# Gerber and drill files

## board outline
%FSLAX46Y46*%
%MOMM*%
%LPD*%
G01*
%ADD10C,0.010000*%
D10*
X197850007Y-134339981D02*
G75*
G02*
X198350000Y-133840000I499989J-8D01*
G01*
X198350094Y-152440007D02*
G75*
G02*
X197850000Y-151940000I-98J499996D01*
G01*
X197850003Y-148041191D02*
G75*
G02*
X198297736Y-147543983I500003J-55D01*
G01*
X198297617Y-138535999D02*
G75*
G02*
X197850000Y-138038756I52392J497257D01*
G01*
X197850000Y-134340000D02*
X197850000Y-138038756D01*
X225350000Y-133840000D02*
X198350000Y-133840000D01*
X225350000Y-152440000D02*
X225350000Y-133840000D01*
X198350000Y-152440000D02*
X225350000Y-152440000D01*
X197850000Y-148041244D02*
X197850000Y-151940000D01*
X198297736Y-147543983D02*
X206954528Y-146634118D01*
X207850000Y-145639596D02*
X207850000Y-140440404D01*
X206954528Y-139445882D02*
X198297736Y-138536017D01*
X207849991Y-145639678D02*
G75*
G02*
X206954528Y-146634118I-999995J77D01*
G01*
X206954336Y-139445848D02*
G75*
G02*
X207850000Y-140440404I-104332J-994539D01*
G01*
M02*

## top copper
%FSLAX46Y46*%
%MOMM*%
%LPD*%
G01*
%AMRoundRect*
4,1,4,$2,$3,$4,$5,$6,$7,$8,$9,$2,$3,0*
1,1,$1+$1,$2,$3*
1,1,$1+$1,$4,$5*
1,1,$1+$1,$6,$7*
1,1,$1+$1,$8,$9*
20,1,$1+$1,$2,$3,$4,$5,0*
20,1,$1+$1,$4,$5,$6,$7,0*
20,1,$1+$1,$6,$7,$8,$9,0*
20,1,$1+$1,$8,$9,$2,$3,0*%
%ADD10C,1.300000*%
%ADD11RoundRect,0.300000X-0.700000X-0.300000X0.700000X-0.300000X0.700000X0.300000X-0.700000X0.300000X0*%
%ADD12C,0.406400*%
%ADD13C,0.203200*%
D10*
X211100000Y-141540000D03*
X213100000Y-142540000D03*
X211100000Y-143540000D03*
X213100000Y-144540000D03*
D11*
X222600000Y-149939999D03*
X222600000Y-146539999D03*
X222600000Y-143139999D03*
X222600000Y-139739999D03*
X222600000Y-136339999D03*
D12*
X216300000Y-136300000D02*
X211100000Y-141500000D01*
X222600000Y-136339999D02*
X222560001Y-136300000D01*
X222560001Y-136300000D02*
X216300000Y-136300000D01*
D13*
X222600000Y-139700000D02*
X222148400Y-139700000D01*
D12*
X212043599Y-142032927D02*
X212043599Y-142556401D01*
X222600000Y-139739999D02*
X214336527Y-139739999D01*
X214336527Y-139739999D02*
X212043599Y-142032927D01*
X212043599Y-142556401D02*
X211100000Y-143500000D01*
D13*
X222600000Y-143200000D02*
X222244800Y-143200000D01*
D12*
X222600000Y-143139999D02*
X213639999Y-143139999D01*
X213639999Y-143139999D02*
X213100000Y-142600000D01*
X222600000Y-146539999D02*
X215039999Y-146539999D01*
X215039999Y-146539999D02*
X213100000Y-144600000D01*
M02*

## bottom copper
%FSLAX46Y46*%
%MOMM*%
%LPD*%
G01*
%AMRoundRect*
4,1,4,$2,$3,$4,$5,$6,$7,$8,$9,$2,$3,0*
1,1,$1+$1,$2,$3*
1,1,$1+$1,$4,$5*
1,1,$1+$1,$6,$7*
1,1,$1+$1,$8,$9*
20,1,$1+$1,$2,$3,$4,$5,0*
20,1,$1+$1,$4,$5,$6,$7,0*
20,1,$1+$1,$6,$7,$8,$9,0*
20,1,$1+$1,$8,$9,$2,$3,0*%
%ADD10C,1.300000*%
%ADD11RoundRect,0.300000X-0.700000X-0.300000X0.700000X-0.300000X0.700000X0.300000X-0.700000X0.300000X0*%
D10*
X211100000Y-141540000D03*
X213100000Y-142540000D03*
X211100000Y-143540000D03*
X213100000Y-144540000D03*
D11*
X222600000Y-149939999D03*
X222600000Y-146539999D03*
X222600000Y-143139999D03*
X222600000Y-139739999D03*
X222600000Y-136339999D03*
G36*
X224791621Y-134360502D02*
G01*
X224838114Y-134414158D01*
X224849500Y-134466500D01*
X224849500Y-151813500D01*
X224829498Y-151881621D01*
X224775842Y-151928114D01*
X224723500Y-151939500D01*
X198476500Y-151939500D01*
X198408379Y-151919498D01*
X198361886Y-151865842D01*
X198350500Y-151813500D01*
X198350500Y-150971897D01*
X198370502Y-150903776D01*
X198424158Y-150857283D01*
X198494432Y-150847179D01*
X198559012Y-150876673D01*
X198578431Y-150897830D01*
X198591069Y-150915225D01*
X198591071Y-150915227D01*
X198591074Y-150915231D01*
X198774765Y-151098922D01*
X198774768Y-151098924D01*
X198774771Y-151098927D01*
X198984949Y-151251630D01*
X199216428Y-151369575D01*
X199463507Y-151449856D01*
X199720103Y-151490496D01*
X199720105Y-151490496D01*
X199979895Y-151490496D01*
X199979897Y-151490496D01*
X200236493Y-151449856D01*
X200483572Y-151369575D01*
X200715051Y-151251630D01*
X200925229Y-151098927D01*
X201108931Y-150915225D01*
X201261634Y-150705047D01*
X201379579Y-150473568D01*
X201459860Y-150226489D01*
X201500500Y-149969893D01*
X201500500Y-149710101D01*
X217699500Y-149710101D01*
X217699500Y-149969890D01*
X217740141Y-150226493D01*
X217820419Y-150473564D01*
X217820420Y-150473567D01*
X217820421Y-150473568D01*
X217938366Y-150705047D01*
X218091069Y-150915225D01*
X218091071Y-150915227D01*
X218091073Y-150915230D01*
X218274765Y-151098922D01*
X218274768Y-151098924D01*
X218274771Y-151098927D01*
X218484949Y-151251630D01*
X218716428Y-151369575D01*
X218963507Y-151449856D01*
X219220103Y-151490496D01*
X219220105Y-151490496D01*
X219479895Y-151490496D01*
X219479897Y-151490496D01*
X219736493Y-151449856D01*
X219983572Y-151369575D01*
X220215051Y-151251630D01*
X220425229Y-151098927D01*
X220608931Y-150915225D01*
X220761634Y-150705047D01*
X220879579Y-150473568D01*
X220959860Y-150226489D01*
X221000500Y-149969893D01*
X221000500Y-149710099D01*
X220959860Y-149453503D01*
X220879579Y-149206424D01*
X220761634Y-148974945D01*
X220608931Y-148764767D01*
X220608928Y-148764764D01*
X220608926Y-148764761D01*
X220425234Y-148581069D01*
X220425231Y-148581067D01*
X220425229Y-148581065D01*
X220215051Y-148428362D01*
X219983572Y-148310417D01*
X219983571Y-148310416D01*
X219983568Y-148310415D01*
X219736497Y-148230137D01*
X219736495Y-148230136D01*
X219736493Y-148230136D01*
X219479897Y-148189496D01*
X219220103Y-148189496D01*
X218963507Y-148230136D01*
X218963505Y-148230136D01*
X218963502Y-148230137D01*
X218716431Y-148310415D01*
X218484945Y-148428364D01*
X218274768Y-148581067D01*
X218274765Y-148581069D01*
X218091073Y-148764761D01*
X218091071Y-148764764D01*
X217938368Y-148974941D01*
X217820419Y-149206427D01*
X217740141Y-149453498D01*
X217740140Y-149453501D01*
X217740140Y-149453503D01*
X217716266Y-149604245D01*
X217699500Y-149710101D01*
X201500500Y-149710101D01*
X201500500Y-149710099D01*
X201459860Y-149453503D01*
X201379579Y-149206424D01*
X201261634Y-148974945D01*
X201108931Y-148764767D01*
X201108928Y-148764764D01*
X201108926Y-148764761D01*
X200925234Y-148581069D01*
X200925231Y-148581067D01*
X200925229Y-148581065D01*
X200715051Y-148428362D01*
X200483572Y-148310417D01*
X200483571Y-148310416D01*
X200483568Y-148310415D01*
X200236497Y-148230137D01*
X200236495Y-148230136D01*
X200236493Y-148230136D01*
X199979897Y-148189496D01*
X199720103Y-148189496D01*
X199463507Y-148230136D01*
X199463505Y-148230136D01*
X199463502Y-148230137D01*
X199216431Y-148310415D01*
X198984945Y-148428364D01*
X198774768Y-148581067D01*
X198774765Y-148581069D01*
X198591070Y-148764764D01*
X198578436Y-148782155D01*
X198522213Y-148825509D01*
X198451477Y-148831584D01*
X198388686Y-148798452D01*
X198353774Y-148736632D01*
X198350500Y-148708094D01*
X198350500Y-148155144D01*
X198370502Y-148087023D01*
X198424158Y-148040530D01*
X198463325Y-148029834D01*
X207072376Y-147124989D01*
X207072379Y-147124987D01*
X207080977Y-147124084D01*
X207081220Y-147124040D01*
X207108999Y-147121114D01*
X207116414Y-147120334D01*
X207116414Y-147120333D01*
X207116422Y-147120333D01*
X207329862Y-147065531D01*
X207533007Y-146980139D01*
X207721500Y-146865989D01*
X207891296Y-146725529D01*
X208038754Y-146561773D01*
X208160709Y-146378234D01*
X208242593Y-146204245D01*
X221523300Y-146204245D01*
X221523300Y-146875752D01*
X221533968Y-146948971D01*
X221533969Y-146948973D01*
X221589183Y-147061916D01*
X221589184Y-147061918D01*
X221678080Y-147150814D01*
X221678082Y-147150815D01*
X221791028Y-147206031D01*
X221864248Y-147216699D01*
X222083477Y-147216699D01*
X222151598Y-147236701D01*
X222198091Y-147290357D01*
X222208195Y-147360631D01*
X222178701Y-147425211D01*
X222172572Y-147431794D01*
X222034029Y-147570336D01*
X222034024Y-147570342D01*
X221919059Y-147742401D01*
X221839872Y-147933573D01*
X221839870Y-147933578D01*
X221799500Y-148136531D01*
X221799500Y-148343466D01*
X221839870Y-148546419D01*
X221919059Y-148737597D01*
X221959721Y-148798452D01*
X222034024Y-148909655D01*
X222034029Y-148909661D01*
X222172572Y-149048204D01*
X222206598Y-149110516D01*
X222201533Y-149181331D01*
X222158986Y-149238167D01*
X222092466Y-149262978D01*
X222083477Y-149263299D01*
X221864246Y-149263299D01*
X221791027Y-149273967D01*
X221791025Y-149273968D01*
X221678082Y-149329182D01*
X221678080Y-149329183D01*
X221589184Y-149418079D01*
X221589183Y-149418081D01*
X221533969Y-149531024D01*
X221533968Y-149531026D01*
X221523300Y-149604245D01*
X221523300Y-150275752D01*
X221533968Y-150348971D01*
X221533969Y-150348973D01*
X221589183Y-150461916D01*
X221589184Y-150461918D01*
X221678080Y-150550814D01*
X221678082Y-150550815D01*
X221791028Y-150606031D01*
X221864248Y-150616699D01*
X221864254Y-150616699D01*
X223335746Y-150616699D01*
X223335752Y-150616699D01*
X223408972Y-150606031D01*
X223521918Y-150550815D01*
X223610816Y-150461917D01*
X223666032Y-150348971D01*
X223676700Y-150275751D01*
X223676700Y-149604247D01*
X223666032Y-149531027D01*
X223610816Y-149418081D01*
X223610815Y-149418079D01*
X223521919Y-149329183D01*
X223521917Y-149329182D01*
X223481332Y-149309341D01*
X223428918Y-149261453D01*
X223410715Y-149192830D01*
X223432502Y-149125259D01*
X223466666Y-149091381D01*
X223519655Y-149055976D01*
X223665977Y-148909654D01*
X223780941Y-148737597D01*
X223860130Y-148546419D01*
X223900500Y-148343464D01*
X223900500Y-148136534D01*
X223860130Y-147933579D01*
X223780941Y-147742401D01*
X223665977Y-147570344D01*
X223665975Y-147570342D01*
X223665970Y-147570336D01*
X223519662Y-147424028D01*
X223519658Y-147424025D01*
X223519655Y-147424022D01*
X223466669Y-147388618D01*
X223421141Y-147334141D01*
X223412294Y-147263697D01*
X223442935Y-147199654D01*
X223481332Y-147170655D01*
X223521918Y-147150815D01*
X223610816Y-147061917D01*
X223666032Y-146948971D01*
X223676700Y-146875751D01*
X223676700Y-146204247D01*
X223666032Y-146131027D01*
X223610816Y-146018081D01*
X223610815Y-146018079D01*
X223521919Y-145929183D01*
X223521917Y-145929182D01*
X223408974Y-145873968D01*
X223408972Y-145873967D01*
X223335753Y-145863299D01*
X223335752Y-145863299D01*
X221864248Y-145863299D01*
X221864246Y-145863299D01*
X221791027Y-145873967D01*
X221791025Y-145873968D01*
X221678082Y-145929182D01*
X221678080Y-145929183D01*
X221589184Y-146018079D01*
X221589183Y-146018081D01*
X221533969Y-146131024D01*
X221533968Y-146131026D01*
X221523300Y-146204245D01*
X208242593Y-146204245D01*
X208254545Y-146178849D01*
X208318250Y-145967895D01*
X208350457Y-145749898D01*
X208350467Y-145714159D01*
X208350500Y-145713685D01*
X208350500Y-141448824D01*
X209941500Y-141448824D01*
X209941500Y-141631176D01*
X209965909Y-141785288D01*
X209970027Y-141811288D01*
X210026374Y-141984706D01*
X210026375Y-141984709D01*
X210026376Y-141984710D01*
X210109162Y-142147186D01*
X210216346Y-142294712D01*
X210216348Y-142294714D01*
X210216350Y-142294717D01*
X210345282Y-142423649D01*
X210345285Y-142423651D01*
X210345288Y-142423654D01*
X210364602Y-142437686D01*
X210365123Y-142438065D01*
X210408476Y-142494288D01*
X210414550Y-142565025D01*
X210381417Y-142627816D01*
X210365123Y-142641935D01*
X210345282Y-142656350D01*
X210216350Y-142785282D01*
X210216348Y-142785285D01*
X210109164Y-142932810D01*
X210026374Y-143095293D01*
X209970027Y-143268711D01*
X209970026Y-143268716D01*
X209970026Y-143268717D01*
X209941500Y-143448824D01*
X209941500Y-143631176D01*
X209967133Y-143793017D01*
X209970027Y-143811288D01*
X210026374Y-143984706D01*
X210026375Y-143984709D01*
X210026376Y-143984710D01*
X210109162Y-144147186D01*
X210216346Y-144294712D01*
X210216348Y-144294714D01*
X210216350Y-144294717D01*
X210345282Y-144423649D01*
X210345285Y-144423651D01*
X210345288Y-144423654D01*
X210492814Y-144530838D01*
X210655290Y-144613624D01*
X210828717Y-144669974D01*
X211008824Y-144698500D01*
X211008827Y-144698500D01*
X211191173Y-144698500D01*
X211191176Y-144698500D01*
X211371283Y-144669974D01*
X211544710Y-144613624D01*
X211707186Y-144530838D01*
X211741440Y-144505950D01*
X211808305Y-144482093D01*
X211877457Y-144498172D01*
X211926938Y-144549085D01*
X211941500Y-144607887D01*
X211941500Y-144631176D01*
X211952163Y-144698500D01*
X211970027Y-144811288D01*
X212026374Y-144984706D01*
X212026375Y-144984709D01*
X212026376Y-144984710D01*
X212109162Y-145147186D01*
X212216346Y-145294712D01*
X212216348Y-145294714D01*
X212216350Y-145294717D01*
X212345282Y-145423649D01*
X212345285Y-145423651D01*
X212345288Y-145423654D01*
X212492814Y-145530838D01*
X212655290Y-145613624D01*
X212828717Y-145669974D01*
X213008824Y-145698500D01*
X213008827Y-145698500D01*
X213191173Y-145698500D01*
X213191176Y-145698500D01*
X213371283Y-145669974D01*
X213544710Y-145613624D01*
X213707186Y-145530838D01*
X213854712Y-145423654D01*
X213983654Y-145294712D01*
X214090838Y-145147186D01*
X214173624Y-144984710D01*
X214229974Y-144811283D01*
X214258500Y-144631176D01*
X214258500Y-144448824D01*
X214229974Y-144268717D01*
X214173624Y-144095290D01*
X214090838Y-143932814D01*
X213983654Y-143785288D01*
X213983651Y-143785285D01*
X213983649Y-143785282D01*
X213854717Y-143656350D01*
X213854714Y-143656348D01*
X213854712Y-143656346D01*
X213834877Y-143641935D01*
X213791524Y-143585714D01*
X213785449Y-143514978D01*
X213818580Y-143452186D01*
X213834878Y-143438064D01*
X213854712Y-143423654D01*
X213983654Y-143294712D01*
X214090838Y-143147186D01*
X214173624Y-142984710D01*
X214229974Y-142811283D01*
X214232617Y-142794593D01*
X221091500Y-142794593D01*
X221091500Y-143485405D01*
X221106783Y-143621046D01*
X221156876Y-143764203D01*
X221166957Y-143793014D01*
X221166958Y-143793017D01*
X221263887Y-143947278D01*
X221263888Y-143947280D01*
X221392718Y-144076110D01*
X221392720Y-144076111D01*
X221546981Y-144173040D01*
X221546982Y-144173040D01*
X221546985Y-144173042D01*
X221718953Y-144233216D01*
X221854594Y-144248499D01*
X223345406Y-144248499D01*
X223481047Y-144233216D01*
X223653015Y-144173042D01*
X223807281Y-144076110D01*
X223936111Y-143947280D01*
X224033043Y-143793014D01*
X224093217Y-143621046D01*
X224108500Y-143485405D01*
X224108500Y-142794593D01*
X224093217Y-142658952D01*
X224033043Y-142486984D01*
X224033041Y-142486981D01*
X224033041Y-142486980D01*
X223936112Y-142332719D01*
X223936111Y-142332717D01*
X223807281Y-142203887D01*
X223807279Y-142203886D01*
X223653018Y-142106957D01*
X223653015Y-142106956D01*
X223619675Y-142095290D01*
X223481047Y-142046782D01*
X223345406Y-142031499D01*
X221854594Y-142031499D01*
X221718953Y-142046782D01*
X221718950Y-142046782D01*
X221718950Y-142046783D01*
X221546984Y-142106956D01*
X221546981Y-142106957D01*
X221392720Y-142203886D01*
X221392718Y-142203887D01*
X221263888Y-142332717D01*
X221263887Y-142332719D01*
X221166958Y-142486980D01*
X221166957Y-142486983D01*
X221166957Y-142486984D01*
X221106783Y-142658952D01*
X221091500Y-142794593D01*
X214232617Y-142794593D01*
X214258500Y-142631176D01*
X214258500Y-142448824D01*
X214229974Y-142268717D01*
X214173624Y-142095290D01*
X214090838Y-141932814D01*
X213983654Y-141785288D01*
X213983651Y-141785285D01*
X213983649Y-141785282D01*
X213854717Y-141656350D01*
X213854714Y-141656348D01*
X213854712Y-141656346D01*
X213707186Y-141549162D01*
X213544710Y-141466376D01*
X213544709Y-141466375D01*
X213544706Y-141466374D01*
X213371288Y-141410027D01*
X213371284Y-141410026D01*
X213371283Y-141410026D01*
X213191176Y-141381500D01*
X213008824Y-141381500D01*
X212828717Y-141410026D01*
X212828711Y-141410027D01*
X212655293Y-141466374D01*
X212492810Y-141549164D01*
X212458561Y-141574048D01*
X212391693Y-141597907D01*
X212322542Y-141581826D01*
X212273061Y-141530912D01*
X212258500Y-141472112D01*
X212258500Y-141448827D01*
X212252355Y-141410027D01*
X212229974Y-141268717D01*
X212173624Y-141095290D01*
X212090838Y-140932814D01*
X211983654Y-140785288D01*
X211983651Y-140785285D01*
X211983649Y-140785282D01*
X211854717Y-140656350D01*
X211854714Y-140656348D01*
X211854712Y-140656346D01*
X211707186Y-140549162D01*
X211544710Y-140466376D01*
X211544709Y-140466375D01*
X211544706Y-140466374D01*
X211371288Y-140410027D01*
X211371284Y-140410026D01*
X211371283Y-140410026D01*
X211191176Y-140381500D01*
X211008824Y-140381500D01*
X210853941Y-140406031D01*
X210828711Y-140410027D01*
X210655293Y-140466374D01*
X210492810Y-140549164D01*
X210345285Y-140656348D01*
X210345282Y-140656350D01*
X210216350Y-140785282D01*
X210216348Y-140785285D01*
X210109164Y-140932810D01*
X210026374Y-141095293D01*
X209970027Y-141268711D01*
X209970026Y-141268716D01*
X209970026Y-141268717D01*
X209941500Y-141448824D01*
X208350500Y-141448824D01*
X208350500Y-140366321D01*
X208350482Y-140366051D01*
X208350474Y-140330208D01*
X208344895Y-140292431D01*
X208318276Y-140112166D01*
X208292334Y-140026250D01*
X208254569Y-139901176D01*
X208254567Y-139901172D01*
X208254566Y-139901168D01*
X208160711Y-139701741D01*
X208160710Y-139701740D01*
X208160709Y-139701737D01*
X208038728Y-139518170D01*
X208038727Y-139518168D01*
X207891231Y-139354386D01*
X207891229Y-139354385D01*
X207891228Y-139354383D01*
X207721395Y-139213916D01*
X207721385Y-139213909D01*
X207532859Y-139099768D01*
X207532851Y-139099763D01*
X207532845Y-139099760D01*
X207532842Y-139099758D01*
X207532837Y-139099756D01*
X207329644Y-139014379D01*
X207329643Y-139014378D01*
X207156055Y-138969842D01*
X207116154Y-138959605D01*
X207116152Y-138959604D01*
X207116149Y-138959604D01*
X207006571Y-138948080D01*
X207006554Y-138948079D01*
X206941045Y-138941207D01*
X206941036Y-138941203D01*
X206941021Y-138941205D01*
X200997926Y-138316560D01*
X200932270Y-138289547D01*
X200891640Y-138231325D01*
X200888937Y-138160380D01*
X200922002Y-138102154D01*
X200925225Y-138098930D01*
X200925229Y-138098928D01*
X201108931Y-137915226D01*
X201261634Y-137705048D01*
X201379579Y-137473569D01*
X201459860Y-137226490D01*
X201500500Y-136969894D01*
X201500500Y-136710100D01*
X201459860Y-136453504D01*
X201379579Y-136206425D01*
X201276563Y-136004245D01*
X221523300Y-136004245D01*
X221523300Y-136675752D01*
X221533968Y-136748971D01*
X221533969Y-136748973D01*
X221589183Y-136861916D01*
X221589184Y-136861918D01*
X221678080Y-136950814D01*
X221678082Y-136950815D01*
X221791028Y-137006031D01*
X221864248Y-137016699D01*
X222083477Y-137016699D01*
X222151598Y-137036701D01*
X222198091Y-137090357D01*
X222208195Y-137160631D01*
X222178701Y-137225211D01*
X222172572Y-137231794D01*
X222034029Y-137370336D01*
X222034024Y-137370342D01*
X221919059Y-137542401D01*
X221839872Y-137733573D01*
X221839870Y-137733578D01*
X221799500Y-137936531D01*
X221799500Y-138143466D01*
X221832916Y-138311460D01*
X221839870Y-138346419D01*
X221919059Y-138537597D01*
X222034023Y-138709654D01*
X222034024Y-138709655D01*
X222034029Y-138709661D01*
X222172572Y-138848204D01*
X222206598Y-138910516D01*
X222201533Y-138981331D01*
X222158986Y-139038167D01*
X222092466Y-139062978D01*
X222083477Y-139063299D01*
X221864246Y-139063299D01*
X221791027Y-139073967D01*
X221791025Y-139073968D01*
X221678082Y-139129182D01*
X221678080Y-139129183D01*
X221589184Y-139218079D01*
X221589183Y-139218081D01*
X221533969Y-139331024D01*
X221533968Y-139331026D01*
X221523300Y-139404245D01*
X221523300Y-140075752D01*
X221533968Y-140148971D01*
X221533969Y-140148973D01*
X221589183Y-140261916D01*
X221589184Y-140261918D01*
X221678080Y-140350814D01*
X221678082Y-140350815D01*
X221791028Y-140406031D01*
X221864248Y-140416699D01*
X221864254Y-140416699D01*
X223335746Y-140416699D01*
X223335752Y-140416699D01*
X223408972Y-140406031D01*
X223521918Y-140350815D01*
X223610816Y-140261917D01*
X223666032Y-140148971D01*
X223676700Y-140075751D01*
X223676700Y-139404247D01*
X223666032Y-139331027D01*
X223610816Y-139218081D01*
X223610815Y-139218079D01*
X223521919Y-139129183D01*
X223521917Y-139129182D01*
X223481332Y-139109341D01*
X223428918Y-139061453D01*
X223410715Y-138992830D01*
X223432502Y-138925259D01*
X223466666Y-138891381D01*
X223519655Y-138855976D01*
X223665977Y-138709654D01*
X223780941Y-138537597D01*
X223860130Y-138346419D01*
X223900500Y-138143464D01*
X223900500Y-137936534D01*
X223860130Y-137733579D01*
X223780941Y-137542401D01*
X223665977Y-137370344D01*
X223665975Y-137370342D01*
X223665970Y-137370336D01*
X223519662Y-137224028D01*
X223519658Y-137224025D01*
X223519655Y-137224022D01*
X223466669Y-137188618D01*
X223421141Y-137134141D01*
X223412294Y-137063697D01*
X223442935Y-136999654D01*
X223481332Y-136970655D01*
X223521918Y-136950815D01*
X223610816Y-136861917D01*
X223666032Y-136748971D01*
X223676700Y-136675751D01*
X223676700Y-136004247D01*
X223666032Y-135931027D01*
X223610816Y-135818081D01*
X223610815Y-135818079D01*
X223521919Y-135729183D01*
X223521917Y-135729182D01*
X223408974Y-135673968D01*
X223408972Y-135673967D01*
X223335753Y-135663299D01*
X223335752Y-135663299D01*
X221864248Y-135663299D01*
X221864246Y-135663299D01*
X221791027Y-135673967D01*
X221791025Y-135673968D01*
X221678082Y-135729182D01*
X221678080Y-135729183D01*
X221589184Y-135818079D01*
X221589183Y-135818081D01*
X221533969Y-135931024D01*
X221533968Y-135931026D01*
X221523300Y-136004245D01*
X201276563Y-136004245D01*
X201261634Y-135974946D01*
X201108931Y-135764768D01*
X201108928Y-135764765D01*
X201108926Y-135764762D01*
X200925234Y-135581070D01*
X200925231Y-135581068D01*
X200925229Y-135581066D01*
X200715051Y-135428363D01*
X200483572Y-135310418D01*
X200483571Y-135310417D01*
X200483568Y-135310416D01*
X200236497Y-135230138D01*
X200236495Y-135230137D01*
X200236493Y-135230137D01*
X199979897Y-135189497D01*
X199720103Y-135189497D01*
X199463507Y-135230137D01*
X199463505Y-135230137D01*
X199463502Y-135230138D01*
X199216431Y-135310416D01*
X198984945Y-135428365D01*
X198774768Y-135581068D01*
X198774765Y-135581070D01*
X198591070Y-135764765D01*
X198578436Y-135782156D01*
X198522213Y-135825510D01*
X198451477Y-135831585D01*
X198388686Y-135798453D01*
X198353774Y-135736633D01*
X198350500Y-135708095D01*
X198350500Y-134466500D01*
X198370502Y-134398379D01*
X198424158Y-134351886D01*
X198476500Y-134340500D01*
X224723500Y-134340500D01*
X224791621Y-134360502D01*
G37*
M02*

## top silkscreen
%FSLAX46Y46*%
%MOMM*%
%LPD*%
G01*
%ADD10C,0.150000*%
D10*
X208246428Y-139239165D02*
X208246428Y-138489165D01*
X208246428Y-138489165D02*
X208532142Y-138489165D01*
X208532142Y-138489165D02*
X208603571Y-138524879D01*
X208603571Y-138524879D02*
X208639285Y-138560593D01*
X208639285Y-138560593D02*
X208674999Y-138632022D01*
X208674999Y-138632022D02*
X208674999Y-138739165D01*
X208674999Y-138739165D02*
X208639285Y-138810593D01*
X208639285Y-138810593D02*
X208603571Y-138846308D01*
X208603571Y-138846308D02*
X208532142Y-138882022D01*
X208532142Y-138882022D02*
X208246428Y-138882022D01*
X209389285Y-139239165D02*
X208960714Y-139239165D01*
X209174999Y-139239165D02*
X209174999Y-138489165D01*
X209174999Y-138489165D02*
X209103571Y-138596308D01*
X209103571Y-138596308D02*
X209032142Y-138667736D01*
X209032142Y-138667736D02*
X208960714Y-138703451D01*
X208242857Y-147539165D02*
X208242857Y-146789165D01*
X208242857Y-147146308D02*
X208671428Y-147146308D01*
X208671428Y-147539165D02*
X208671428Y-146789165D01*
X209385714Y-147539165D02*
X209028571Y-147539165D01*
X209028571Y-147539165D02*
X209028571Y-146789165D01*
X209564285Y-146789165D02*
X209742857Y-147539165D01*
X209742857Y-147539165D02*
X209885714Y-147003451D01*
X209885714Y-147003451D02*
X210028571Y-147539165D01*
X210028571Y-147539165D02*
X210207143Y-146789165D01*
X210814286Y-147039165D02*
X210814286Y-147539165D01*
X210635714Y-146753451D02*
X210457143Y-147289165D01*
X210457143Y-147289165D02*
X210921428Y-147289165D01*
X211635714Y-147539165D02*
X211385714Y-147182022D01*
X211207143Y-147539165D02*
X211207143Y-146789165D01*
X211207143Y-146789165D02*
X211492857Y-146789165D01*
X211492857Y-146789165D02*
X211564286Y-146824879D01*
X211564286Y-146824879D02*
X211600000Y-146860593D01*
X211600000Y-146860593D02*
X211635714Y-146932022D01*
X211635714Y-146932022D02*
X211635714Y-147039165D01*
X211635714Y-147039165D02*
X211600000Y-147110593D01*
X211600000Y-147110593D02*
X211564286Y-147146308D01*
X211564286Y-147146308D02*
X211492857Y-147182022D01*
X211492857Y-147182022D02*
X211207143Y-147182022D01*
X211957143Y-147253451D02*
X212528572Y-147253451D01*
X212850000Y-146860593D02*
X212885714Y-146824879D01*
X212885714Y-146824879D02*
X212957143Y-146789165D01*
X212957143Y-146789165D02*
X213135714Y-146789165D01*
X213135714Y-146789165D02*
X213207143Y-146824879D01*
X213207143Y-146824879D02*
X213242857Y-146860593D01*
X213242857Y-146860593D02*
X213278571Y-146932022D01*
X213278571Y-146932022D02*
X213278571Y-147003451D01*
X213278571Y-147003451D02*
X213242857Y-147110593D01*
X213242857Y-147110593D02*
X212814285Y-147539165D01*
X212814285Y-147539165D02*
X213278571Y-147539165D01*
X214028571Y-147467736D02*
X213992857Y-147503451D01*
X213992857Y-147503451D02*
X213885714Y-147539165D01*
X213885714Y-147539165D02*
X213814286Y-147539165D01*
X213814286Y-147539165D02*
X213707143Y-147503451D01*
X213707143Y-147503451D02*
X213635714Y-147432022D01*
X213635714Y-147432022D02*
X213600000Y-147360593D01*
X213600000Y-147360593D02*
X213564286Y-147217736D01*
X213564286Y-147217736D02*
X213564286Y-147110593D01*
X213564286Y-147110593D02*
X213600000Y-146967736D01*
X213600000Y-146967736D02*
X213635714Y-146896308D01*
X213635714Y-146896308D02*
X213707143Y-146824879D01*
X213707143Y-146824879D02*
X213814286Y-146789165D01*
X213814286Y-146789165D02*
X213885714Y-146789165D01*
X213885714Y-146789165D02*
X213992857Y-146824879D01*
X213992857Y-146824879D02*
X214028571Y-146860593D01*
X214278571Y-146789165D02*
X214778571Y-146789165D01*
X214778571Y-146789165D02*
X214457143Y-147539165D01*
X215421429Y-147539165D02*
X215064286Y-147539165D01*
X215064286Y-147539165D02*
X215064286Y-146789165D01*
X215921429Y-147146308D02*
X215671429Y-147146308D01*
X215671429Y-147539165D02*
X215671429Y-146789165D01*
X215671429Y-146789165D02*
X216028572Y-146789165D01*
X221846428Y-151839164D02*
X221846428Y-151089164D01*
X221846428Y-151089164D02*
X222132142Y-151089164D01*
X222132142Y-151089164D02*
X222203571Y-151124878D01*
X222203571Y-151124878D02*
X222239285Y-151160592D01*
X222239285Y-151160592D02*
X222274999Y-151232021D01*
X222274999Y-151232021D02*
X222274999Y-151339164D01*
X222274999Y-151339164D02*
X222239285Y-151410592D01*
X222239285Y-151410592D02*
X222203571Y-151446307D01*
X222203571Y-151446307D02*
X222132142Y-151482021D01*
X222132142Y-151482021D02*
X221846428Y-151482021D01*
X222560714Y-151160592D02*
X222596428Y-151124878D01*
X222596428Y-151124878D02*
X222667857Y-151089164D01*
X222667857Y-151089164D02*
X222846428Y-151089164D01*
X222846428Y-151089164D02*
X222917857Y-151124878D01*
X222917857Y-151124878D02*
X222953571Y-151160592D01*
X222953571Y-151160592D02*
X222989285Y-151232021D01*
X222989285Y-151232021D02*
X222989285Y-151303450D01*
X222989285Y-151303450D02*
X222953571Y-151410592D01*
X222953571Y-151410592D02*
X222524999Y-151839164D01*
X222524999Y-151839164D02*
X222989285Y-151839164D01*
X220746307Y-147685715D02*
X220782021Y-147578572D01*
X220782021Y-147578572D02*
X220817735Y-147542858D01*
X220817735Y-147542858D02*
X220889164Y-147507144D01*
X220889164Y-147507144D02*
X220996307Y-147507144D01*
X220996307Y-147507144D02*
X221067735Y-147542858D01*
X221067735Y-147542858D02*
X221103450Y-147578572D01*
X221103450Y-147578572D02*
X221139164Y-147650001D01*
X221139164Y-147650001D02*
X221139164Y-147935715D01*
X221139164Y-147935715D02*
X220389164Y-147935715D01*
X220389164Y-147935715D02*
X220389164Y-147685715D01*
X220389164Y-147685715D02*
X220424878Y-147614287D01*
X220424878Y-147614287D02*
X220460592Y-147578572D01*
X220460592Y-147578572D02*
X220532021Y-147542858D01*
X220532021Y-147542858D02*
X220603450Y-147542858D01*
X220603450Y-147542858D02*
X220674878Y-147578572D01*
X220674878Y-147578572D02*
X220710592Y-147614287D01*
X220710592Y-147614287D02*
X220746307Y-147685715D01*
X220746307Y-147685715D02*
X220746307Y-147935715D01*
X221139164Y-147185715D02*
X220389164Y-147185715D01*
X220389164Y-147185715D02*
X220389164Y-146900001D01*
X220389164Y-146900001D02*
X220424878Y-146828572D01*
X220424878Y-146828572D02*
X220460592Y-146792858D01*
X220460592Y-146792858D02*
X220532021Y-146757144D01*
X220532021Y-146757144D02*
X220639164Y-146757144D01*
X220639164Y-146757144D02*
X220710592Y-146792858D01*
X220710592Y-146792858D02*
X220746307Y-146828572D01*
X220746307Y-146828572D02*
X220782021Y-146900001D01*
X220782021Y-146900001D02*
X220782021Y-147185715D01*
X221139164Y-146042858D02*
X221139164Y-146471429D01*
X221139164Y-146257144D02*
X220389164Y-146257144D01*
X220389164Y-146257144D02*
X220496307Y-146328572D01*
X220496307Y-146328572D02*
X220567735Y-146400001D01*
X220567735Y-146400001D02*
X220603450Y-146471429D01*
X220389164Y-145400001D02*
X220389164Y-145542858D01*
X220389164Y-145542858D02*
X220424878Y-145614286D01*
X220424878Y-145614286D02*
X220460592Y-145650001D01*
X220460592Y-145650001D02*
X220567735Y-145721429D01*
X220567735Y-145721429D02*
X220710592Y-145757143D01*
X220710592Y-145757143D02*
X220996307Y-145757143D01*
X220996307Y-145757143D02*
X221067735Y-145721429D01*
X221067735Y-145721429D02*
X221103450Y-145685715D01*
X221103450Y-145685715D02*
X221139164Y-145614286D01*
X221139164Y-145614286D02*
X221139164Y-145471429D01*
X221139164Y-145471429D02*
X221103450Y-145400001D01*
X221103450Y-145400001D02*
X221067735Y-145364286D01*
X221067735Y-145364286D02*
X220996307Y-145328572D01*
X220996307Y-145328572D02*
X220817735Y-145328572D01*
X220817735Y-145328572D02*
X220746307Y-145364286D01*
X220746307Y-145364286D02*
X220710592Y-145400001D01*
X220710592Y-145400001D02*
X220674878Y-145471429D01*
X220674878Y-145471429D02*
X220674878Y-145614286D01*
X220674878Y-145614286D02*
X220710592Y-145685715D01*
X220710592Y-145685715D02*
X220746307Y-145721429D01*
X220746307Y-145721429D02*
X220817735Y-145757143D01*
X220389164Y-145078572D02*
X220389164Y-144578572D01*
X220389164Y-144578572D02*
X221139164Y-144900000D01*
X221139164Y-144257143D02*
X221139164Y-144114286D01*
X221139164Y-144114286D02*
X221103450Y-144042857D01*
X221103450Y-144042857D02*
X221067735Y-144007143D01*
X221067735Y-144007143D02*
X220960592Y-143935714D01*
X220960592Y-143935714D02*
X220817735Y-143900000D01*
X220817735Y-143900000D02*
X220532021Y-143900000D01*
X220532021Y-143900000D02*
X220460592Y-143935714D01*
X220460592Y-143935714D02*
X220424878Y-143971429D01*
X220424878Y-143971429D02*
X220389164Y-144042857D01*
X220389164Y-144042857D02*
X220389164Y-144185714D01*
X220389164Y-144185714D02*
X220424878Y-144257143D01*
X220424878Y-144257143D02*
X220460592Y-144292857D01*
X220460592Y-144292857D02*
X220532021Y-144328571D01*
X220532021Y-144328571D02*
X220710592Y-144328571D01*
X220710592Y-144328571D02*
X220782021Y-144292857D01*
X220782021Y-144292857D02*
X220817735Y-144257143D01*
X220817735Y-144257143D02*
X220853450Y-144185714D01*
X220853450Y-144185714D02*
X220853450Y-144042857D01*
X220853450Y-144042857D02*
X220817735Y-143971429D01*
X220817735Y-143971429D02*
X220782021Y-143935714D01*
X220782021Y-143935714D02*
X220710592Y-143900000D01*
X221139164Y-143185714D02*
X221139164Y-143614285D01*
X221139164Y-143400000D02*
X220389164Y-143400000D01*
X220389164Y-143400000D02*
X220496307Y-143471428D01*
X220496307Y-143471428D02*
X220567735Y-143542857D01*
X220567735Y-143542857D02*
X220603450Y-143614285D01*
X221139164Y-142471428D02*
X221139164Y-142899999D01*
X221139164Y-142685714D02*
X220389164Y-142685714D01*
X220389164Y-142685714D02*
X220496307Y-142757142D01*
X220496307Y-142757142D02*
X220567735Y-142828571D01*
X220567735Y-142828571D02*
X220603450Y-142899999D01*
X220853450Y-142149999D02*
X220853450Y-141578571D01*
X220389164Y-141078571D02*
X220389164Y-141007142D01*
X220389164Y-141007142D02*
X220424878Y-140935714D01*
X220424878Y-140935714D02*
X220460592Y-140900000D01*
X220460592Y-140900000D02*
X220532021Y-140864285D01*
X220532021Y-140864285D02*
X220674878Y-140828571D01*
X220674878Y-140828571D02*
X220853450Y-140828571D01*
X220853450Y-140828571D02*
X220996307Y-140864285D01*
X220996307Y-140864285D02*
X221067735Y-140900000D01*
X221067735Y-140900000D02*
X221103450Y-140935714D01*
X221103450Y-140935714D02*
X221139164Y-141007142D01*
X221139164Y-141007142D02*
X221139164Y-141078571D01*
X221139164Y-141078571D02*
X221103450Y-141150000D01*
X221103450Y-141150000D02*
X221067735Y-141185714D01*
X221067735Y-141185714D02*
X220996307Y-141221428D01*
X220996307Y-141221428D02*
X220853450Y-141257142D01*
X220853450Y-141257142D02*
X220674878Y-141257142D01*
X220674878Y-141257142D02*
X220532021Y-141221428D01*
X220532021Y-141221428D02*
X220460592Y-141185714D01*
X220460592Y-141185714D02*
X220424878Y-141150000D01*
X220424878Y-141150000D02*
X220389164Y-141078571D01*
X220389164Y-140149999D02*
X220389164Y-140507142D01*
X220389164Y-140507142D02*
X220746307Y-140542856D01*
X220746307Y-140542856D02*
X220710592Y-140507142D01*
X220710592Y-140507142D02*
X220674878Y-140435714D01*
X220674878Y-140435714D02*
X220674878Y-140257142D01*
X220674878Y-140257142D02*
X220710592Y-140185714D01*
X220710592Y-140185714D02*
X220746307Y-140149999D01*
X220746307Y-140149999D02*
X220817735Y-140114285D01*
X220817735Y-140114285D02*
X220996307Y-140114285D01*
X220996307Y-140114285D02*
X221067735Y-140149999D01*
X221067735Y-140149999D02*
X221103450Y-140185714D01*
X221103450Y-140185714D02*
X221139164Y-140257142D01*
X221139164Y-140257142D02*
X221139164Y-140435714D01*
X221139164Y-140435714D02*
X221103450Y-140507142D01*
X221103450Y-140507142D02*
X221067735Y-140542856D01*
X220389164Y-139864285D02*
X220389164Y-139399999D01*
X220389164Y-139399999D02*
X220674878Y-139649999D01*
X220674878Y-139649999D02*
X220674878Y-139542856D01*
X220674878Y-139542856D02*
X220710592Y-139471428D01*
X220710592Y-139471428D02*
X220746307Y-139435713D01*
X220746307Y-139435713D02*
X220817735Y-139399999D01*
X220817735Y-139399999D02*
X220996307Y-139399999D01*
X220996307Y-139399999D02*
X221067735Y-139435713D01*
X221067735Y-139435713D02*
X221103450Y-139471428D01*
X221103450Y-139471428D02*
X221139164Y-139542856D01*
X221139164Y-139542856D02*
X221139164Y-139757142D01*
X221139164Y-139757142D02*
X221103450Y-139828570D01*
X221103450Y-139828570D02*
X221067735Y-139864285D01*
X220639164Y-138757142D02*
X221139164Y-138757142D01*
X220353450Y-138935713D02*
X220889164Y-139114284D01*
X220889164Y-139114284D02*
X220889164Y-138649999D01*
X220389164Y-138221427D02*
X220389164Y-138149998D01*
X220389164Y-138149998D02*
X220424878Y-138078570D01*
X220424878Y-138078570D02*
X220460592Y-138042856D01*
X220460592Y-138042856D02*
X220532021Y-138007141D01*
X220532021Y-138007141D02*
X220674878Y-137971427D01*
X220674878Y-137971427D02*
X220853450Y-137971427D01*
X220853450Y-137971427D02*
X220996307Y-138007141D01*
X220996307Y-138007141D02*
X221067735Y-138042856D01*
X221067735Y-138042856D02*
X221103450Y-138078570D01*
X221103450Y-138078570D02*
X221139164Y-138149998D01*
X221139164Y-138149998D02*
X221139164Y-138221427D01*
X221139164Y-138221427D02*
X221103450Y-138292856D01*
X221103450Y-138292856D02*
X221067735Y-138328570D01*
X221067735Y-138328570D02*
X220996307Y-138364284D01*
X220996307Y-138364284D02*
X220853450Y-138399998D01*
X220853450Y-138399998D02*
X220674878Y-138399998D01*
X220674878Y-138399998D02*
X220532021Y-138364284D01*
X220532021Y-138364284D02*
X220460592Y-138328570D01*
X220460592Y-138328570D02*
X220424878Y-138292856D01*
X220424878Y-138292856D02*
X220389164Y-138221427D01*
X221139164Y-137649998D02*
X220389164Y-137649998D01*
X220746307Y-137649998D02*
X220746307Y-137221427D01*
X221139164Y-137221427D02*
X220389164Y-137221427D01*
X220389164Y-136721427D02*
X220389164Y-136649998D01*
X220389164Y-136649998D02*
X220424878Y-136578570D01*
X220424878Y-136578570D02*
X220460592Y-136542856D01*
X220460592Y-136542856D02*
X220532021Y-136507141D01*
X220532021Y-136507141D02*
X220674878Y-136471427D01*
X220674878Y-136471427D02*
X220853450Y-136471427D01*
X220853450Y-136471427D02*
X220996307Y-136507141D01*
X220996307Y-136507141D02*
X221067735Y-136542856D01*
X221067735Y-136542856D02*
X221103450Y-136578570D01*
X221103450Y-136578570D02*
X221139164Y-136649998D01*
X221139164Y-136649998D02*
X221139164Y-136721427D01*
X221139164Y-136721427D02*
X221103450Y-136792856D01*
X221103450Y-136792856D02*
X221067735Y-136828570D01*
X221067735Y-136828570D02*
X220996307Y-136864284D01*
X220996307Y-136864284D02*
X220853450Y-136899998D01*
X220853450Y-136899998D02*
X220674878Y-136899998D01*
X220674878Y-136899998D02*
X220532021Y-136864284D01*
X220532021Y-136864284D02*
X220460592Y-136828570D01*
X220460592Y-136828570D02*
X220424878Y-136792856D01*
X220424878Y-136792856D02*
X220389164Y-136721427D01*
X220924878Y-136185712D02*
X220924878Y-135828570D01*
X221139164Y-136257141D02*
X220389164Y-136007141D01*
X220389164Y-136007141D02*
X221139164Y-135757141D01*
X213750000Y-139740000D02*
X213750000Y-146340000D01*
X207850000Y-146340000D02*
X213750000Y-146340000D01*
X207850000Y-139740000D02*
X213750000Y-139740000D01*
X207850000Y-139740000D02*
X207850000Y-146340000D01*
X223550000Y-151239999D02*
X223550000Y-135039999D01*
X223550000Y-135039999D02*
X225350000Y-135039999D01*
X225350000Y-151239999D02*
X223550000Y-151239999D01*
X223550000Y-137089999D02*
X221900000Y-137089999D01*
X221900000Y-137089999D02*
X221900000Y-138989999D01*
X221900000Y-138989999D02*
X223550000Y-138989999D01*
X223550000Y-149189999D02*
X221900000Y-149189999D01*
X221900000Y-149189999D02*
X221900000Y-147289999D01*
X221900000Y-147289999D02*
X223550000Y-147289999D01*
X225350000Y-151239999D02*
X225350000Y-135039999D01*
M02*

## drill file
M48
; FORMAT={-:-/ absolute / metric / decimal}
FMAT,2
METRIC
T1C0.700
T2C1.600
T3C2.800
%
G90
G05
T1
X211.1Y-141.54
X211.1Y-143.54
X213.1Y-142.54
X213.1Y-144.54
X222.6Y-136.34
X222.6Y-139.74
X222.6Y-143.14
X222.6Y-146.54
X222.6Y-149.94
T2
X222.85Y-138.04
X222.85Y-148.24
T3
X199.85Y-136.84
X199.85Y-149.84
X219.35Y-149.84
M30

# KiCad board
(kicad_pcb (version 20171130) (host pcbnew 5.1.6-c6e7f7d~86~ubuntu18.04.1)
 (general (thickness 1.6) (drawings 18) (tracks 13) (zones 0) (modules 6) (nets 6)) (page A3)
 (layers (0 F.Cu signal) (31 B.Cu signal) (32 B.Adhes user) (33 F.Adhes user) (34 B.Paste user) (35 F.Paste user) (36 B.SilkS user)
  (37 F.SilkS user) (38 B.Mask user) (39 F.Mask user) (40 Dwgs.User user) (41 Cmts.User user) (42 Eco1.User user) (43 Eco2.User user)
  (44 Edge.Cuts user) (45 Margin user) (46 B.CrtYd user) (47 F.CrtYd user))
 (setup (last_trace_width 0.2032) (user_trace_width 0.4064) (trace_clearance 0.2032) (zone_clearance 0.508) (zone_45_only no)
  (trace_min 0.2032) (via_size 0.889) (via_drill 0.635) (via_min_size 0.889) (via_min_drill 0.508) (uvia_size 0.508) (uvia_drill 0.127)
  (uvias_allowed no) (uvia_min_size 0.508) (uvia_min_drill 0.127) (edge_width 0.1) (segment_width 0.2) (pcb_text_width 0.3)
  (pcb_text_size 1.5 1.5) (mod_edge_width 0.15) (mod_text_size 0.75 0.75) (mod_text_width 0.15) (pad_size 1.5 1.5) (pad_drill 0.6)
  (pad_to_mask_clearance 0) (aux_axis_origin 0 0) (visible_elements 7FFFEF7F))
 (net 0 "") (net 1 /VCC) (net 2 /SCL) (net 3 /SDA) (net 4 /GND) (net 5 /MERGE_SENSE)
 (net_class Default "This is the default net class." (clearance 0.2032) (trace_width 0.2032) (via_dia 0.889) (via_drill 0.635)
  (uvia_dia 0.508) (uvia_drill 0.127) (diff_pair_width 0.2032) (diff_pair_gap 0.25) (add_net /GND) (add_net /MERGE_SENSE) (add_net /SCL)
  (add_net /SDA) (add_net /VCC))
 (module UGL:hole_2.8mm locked (layer F.Cu) (at 219.35 149.839996)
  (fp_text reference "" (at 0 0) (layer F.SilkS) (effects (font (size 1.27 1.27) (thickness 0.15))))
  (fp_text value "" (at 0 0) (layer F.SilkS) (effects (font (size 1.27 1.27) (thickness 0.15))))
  (pad "" np_thru_hole circle (at 0 0) (size 2.8 2.8) (drill 2.8) (layers *.Cu *.Mask)))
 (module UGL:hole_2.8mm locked (layer F.Cu) (at 199.85 149.839996)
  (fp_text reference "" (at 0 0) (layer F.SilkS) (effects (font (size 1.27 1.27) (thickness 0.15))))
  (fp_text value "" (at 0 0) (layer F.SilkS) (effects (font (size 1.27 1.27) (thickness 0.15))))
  (pad "" np_thru_hole circle (at 0 0) (size 2.8 2.8) (drill 2.8) (layers *.Cu *.Mask)))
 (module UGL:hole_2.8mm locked (layer F.Cu) (at 199.85 136.839997)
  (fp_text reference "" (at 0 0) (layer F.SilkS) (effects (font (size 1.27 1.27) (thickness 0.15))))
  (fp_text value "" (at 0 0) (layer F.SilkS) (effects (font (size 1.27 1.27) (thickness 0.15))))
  (pad "" np_thru_hole circle (at 0 0) (size 2.8 2.8) (drill 2.8) (layers *.Cu *.Mask)))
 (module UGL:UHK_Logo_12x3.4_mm (layer B.Cu) (at 209.6 149.7 180)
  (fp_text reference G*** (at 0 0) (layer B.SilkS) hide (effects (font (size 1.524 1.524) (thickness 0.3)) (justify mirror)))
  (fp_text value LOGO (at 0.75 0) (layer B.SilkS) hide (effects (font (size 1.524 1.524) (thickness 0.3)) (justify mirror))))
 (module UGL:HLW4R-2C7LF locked (layer F.Cu) (at 207.85 143.04 270)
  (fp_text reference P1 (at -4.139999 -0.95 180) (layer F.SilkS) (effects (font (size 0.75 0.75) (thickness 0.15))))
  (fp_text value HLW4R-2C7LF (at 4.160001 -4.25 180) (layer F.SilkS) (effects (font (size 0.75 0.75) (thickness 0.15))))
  (fp_line (start -3.3 -5.9) (end 3.3 -5.9) (layer F.SilkS) (width 0.15))
  (fp_line (start 3.3 0) (end 3.3 -5.9) (layer F.SilkS) (width 0.15))
  (fp_line (start -3.3 0) (end -3.3 -5.9) (layer F.SilkS) (width 0.15))
  (fp_line (start -3.3 0) (end 3.3 0) (layer F.SilkS) (width 0.15))
  (pad 4 thru_hole circle (at -1.5 -3.25 270) (size 1.3 1.3) (drill 0.7) (layers *.Cu *.Mask) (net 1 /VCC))
  (pad 3 thru_hole circle (at -0.5 -5.25 270) (size 1.3 1.3) (drill 0.7) (layers *.Cu *.Mask) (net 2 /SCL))
  (pad 2 thru_hole circle (at 0.5 -3.25 270) (size 1.3 1.3) (drill 0.7) (layers *.Cu *.Mask) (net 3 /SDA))
  (pad 1 thru_hole circle (at 1.5 -5.25 270) (size 1.3 1.3) (drill 0.7) (layers *.Cu *.Mask) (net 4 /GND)))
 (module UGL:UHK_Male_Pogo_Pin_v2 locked (layer F.Cu) (at 225.35 143.139999)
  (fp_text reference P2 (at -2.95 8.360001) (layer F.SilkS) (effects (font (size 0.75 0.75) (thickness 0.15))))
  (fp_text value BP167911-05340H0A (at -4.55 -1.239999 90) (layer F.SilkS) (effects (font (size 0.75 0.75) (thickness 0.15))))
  (fp_line (start -1.8 8.1) (end -1.8 -8.1) (layer F.SilkS) (width 0.15))
  (fp_line (start -1.8 -8.1) (end 0 -8.1) (layer F.SilkS) (width 0.15))
  (fp_line (start 0 8.1) (end -1.8 8.1) (layer F.SilkS) (width 0.15))
  (fp_line (start -1.8 -6.05) (end -3.45 -6.05) (layer F.SilkS) (width 0.15))
  (fp_line (start -3.45 -6.05) (end -3.45 -4.15) (layer F.SilkS) (width 0.15))
  (fp_line (start -3.45 -4.15) (end -1.8 -4.15) (layer F.SilkS) (width 0.15))
  (fp_line (start -1.8 6.05) (end -3.45 6.05) (layer F.SilkS) (width 0.15))
  (fp_line (start -3.45 6.05) (end -3.45 4.15) (layer F.SilkS) (width 0.15))
  (fp_line (start -3.45 4.15) (end -1.8 4.15) (layer F.SilkS) (width 0.15))
  (fp_line (start 0 8.1) (end 0 -8.1) (layer F.SilkS) (width 0.15))
  (pad "" np_thru_hole circle (at -2.5 5.1 180) (size 1.6 1.6) (drill 1.6) (layers *.Cu *.Mask) (clearance 0.00254))
  (pad "" np_thru_hole circle (at -2.5 -5.1) (size 1.6 1.6) (drill 1.6) (layers *.Cu *.Mask) (clearance 0.00254))
  (pad 5 thru_hole roundrect (at -2.75 6.8) (size 2 1.2) (drill 0.7) (layers *.Cu *.Mask) (roundrect_rratio 0.25) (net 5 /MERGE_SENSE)
   (clearance 0.0762))
  (pad 4 thru_hole roundrect (at -2.75 3.4) (size 2 1.2) (drill 0.7) (layers *.Cu *.Mask) (roundrect_rratio 0.25) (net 4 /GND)
   (clearance 0.0762))
  (pad 3 thru_hole roundrect (at -2.75 0) (size 2 1.2) (drill 0.7) (layers *.Cu *.Mask) (roundrect_rratio 0.25) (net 2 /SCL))
  (pad 2 thru_hole roundrect (at -2.75 -3.4) (size 2 1.2) (drill 0.7) (layers *.Cu *.Mask) (roundrect_rratio 0.25) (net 3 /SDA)
   (clearance 0.0762))
  (pad 1 thru_hole roundrect (at -2.75 -6.8) (size 2 1.2) (drill 0.7) (layers *.Cu *.Mask) (roundrect_rratio 0.25) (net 1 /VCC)
   (clearance 0.0762)))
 (gr_arc (start 198.349996 134.339989) (end 198.35 133.84) (angle -89.99948442) (layer Edge.Cuts) (width 0.01))
 (gr_arc (start 198.349996 151.940011) (end 197.85 151.94) (angle -90.01245443) (layer Edge.Cuts) (width 0.01))
 (gr_arc (start 198.350006 148.041246) (end 198.297736 147.543983) (angle -83.99301623) (layer Edge.Cuts) (width 0.01))
 (gr_arc (start 198.350009 138.038742) (end 197.85 138.038756) (angle -83.98380083) (layer Edge.Cuts) (width 0.01))
 (gr_line (start 197.85 134.34) (end 197.85 138.038756) (angle 90) (layer Edge.Cuts) (width 0.01))
 (gr_line (start 225.35 133.84) (end 198.35 133.84) (angle 90) (layer Edge.Cuts) (width 0.01))
 (gr_line (start 225.35 152.44) (end 225.35 133.84) (angle 90) (layer Edge.Cuts) (width 0.01))
 (gr_line (start 198.35 152.44) (end 225.35 152.44) (angle 90) (layer Edge.Cuts) (width 0.01))
 (gr_line (start 197.85 148.041244) (end 197.85 151.94) (angle 90) (layer Edge.Cuts) (width 0.01))
 (gr_line (start 198.297736 147.543983) (end 206.954528 146.634118) (angle 90) (layer Edge.Cuts) (width 0.01))
 (gr_line (start 207.85 145.639596) (end 207.85 140.440404) (angle 90) (layer Edge.Cuts) (width 0.01))
 (gr_line (start 206.954528 139.445882) (end 198.297736 138.536017) (angle 90) (layer Edge.Cuts) (width 0.01))
 (gr_arc (start 206.849996 145.639601) (end 206.954528 146.634118) (angle -83.99535087) (layer Edge.Cuts) (width 0.01))
 (gr_arc (start 206.850004 140.440387) (end 207.85 140.440404) (angle -84.01229189) (layer Edge.Cuts) (width 0.01))
 (segment (start 216.3 136.3) (end 211.1 141.5) (width 0.4064) (layer F.Cu) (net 1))
 (segment (start 222.6 136.339999) (end 222.560001 136.3) (width 0.4064) (layer F.Cu) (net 1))
 (segment (start 222.560001 136.3) (end 216.3 136.3) (width 0.4064) (layer F.Cu) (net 1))
 (segment (start 222.6 139.7) (end 222.1484 139.7) (width 0.2032) (layer F.Cu) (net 3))
 (segment (start 212.043599 142.032927) (end 212.043599 142.556401) (width 0.4064) (layer F.Cu) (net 3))
 (segment (start 222.6 139.739999) (end 214.336527 139.739999) (width 0.4064) (layer F.Cu) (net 3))
 (segment (start 214.336527 139.739999) (end 212.043599 142.032927) (width 0.4064) (layer F.Cu) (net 3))
 (segment (start 212.043599 142.556401) (end 211.1 143.5) (width 0.4064) (layer F.Cu) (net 3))
 (segment (start 222.6 143.2) (end 222.2448 143.2) (width 0.2032) (layer F.Cu) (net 2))
 (segment (start 222.6 143.139999) (end 213.639999 143.139999) (width 0.4064) (layer F.Cu) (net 2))
 (segment (start 213.639999 143.139999) (end 213.1 142.6) (width 0.4064) (layer F.Cu) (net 2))
 (segment (start 222.6 146.539999) (end 215.039999 146.539999) (width 0.4064) (layer F.Cu) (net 4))
 (segment (start 215.039999 146.539999) (end 213.1 144.6) (width 0.4064) (layer F.Cu) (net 4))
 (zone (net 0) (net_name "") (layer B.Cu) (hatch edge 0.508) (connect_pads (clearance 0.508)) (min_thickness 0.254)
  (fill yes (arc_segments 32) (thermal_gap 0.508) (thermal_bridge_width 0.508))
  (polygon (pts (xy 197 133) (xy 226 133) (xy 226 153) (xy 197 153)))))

